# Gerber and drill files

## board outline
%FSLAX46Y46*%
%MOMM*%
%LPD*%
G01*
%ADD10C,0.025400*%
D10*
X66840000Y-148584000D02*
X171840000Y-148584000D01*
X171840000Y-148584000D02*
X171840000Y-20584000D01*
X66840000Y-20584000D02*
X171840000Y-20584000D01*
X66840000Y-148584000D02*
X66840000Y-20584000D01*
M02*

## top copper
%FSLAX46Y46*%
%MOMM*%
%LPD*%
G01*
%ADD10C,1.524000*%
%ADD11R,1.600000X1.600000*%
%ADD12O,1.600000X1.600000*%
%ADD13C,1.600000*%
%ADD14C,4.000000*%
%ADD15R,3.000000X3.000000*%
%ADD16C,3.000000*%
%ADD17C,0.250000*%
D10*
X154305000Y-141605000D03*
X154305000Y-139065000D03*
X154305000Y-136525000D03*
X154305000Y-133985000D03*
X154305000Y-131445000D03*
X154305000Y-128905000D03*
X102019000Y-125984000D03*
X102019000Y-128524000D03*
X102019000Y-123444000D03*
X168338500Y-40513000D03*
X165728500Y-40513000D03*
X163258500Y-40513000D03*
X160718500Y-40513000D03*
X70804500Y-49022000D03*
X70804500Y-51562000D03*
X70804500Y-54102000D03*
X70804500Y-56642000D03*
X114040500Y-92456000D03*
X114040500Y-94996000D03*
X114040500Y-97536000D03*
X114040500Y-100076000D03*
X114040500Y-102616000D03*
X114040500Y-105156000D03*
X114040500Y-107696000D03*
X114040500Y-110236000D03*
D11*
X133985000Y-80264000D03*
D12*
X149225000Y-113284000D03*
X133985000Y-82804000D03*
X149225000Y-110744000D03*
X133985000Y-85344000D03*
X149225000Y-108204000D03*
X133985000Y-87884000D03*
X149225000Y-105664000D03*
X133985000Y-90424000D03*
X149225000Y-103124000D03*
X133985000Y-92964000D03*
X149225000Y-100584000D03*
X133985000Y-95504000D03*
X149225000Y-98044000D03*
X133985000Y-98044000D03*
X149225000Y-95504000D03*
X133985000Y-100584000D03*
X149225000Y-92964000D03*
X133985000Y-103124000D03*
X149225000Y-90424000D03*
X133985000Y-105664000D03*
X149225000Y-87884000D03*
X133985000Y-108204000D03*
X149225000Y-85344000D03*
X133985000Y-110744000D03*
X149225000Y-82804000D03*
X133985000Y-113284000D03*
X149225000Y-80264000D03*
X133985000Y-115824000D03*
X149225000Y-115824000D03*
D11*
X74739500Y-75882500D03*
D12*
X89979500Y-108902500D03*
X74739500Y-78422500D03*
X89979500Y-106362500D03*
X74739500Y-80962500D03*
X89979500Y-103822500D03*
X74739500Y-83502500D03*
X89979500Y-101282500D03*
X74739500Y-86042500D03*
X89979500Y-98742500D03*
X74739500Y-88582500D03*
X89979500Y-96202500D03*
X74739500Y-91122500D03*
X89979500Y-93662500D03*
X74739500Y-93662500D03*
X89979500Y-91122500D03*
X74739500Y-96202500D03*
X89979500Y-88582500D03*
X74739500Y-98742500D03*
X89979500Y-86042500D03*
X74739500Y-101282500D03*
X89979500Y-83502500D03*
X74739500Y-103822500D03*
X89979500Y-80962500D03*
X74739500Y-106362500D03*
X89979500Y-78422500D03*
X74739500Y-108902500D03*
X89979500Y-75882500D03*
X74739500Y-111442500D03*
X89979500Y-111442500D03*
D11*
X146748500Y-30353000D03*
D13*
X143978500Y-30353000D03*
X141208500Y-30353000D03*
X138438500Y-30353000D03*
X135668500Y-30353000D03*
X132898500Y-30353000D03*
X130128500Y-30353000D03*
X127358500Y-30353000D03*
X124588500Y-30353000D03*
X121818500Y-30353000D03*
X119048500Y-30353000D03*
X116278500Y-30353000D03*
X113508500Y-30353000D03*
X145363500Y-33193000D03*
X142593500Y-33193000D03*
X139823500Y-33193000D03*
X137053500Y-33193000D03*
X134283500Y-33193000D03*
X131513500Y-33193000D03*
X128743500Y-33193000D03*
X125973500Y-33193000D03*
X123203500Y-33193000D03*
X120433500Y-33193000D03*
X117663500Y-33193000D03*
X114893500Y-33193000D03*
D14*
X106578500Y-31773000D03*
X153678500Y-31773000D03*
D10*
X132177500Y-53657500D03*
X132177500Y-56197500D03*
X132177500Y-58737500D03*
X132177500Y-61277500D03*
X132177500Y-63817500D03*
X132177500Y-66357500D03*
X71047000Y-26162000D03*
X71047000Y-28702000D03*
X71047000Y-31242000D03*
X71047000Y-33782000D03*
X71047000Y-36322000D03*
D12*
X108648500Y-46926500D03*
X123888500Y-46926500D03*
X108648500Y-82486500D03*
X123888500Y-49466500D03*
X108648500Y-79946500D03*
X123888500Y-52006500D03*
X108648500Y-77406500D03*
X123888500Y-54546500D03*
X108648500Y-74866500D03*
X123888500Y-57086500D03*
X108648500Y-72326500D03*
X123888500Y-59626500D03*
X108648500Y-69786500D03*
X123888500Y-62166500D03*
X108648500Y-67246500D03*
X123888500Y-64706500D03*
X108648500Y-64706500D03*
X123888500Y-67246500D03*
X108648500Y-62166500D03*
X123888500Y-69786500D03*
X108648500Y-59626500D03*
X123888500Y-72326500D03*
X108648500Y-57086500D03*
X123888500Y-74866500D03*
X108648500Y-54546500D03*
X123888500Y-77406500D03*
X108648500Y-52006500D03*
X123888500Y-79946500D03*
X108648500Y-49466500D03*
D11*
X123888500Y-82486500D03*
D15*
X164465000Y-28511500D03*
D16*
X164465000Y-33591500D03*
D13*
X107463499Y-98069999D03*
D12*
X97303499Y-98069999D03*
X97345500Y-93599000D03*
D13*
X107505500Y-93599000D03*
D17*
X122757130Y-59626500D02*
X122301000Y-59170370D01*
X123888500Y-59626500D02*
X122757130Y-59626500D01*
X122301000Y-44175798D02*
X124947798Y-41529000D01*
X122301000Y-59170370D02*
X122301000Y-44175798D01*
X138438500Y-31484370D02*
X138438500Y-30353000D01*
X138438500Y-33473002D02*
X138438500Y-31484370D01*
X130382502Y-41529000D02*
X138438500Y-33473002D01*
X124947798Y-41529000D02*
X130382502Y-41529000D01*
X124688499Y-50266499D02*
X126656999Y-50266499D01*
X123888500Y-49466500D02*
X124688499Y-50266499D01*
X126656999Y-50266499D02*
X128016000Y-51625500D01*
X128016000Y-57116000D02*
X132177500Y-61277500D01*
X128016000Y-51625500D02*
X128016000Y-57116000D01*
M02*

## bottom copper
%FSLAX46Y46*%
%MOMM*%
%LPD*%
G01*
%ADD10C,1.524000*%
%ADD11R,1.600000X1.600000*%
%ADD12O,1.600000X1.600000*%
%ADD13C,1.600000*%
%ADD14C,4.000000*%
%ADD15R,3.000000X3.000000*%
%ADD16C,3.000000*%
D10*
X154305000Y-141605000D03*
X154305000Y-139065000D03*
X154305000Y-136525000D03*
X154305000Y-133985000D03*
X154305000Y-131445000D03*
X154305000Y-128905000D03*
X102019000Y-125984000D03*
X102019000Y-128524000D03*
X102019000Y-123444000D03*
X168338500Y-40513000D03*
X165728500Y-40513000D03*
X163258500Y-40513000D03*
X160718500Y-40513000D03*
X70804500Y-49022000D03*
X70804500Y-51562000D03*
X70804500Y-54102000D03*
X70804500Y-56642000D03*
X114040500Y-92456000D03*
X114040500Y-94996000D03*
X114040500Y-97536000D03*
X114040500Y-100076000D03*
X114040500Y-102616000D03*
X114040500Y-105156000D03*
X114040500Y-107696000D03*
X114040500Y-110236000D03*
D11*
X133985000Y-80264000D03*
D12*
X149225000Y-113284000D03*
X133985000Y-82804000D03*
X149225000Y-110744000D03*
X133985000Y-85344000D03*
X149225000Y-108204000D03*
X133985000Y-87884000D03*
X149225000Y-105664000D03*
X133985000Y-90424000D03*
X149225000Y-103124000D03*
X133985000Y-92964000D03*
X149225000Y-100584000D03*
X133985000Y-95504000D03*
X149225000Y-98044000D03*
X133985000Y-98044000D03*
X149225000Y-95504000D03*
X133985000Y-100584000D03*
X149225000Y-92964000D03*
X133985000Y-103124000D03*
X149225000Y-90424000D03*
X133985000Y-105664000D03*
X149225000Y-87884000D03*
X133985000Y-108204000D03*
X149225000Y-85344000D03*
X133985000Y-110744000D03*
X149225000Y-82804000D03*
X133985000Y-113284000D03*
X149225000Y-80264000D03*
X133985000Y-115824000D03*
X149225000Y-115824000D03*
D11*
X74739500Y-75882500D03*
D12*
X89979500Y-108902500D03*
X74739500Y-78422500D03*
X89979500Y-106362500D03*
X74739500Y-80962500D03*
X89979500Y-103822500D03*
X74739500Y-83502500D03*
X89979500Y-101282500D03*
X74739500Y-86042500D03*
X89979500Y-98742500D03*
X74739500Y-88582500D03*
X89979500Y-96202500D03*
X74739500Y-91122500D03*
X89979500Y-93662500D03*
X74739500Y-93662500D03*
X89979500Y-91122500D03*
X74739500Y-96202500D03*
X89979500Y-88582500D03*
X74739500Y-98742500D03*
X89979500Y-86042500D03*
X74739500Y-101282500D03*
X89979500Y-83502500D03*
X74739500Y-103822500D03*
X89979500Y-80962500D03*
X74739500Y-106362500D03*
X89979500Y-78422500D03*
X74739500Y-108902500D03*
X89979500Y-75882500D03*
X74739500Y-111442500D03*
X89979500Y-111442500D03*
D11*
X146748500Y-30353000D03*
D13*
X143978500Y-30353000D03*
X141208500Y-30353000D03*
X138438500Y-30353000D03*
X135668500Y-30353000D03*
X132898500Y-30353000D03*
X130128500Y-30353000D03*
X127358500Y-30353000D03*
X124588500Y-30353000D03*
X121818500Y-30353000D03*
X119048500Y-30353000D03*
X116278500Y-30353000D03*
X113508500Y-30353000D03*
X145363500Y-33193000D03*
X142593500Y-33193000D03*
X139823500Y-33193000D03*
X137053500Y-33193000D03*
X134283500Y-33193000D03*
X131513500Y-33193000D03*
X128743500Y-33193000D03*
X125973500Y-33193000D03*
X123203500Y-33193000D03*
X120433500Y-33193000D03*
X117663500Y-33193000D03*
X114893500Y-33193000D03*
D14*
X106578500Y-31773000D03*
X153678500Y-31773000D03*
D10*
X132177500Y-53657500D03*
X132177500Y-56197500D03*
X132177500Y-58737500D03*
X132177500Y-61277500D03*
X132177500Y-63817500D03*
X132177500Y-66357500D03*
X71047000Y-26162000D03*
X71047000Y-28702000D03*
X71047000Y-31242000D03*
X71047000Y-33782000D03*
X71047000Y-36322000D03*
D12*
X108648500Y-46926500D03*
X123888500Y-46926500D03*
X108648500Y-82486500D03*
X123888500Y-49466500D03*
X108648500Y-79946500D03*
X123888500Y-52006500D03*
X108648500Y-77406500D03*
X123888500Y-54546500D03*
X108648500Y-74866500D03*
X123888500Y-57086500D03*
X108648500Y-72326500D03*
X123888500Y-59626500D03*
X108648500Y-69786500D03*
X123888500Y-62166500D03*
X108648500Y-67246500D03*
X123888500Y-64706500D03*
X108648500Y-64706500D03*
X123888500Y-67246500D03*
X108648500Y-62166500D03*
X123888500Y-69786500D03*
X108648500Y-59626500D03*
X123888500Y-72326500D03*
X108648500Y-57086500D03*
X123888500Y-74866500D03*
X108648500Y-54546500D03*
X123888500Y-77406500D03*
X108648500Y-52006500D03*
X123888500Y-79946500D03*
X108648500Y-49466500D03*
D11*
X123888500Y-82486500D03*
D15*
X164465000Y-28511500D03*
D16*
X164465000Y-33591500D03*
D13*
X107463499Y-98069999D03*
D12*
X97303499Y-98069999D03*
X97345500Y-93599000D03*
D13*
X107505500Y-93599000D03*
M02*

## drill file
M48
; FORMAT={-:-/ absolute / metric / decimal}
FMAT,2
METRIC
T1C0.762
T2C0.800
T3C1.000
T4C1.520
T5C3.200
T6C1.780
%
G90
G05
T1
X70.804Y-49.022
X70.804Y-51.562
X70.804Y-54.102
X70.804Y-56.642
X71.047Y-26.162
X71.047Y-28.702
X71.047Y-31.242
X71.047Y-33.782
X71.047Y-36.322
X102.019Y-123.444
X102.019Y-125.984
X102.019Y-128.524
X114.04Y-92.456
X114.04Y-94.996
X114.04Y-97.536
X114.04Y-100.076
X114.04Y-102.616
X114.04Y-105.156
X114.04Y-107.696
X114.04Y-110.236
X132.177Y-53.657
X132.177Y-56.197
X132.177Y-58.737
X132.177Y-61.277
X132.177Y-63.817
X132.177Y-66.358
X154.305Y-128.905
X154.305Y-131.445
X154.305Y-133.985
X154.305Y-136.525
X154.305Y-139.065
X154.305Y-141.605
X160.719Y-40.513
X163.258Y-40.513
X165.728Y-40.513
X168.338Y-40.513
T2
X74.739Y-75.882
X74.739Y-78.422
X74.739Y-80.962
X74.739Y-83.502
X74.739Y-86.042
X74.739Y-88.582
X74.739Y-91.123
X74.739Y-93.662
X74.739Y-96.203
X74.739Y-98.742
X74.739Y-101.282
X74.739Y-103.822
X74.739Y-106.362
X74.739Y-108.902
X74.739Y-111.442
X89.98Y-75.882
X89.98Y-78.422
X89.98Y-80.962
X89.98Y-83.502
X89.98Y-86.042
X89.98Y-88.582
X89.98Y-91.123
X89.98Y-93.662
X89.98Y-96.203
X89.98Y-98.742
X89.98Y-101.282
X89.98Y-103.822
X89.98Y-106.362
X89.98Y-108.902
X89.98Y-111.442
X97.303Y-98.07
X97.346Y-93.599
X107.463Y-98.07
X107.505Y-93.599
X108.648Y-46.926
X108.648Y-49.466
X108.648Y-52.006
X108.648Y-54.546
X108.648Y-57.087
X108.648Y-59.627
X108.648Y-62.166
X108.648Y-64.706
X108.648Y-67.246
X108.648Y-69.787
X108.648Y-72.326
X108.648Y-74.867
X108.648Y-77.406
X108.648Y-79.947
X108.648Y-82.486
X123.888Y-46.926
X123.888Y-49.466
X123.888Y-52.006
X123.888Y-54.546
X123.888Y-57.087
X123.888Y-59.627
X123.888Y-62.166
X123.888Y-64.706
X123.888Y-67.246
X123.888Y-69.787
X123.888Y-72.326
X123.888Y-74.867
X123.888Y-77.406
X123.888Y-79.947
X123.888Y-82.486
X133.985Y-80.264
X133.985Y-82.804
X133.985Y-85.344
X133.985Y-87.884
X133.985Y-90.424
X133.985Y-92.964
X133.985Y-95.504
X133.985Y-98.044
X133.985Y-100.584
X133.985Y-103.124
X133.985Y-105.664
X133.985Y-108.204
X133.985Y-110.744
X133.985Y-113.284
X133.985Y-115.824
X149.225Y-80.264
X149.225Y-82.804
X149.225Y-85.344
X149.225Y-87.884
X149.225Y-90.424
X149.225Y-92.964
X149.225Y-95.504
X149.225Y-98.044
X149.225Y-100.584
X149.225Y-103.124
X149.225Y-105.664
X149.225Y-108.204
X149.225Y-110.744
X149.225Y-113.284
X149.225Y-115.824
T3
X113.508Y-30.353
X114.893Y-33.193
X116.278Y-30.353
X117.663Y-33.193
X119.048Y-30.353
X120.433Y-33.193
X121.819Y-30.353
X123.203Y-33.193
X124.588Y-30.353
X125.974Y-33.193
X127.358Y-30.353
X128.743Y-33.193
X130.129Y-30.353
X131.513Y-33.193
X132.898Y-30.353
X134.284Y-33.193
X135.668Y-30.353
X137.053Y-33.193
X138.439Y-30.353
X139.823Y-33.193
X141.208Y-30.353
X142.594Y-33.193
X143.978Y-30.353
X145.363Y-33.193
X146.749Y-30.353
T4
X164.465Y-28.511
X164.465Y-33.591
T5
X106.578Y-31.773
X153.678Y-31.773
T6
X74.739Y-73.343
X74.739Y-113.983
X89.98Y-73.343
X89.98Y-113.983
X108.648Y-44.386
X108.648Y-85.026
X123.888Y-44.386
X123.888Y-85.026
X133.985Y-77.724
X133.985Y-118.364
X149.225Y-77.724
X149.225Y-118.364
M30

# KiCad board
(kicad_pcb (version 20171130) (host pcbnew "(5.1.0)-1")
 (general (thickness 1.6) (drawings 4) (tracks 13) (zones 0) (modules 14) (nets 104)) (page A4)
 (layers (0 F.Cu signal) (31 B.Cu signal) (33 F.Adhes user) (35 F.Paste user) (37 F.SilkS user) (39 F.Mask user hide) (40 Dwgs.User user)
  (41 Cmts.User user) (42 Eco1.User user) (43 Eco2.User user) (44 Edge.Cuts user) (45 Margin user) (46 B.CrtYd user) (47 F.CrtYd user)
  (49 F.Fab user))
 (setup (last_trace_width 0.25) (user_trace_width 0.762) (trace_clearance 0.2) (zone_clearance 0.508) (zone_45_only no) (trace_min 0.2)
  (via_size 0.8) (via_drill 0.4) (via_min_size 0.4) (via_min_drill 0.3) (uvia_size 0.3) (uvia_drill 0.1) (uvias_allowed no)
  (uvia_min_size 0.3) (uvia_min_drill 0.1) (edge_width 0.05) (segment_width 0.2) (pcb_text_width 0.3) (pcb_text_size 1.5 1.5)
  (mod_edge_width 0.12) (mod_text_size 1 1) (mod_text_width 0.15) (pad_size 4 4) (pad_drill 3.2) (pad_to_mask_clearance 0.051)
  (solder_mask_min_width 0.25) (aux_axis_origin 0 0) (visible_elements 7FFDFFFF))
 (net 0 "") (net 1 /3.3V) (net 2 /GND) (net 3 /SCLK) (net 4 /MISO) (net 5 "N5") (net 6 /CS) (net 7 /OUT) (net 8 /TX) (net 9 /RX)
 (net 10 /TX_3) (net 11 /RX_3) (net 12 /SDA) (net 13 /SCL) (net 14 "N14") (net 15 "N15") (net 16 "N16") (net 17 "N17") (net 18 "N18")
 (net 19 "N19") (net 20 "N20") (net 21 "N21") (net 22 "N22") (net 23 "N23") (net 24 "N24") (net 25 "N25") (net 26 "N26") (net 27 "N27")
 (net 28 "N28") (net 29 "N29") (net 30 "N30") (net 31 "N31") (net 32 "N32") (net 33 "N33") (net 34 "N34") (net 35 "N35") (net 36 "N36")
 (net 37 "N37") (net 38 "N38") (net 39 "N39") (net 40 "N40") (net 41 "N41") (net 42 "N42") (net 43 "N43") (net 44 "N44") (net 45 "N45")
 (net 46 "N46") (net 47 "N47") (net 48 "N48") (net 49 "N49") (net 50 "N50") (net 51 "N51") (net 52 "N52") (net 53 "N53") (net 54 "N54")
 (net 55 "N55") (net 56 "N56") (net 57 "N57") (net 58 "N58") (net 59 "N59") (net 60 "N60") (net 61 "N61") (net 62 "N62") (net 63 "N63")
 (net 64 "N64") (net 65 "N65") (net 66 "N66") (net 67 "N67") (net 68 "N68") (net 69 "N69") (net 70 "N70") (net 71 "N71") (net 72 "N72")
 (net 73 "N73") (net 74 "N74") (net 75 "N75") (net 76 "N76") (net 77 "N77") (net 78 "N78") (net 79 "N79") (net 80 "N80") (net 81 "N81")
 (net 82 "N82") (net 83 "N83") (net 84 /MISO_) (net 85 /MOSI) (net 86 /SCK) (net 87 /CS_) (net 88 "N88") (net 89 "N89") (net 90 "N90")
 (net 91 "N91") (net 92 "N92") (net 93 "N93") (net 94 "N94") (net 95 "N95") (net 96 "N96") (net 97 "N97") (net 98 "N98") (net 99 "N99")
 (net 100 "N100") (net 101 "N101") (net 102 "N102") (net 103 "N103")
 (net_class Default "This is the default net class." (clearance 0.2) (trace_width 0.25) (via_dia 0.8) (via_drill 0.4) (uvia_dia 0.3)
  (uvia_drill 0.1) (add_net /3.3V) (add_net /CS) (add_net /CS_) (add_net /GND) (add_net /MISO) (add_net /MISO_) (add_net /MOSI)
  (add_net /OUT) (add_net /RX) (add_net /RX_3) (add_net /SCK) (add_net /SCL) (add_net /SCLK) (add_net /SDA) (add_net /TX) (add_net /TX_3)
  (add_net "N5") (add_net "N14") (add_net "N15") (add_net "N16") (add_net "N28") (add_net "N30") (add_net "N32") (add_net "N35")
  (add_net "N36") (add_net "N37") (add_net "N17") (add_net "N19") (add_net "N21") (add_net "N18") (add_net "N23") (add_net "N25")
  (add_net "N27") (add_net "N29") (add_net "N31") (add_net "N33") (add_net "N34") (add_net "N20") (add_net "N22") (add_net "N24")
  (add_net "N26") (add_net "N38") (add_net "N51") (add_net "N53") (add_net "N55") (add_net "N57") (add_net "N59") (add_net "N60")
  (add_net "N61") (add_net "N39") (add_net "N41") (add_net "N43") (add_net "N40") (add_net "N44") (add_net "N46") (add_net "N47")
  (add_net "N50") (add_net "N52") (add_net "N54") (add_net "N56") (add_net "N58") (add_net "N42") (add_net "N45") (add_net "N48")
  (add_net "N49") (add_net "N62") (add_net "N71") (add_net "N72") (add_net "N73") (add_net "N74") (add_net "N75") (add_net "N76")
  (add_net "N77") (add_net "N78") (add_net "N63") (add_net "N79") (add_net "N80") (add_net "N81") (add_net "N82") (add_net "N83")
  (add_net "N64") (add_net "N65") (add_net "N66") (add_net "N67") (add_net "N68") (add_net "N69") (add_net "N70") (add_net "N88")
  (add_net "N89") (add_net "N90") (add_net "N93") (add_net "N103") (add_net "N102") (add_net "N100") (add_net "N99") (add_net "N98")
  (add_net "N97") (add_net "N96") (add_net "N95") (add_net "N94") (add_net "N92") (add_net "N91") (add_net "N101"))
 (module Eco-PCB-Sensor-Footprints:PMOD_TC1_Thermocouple (layer F.Cu) (at 150.495 137.795 90)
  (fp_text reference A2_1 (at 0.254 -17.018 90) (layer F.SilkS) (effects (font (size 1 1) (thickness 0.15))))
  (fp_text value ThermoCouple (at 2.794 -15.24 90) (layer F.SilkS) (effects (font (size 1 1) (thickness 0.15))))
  (pad 1 thru_hole circle (at -3.81 3.81 90) (size 1.524 1.524) (drill 0.762) (layers *.Cu *.Mask) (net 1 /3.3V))
  (pad 2 thru_hole circle (at -1.27 3.81 90) (size 1.524 1.524) (drill 0.762) (layers *.Cu *.Mask) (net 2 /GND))
  (pad 3 thru_hole circle (at 1.27 3.81 90) (size 1.524 1.524) (drill 0.762) (layers *.Cu *.Mask) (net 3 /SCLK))
  (pad 4 thru_hole circle (at 3.81 3.81 90) (size 1.524 1.524) (drill 0.762) (layers *.Cu *.Mask) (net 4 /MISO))
  (pad 5 thru_hole circle (at 6.35 3.81 90) (size 1.524 1.524) (drill 0.762) (layers *.Cu *.Mask) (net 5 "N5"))
  (pad 6 thru_hole circle (at 8.89 3.81 90) (size 1.524 1.524) (drill 0.762) (layers *.Cu *.Mask) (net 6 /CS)))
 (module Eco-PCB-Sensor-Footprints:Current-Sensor (layer F.Cu) (at 88.519 125.984 90)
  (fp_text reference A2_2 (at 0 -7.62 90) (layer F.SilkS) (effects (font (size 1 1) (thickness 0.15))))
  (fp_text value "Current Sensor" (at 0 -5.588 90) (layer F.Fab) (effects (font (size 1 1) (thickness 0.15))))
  (pad 2 thru_hole circle (at 0 13.5 90) (size 1.524 1.524) (drill 0.762) (layers *.Cu *.Mask) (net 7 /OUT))
  (pad 1 thru_hole circle (at -2.54 13.5 90) (size 1.524 1.524) (drill 0.762) (layers *.Cu *.Mask) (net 1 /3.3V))
  (pad 3 thru_hole circle (at 2.54 13.5 90) (size 1.524 1.524) (drill 0.762) (layers *.Cu *.Mask) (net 2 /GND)))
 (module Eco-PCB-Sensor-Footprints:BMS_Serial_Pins (layer F.Cu) (at 164.5285 40.513 180)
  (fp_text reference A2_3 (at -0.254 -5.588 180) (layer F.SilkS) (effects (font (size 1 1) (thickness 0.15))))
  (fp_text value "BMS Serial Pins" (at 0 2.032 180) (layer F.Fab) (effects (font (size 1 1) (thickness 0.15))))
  (pad 1 thru_hole circle (at -3.81 0 180) (size 1.524 1.524) (drill 0.762) (layers *.Cu *.Mask) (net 1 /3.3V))
  (pad 2 thru_hole circle (at -1.2 0 180) (size 1.524 1.524) (drill 0.762) (layers *.Cu *.Mask) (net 2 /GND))
  (pad 3 thru_hole circle (at 1.27 0 180) (size 1.524 1.524) (drill 0.762) (layers *.Cu *.Mask) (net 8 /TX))
  (pad 4 thru_hole circle (at 3.81 0 180) (size 1.524 1.524) (drill 0.762) (layers *.Cu *.Mask) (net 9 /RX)))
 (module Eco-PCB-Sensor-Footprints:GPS (layer F.Cu) (at 86.8045 52.832 270)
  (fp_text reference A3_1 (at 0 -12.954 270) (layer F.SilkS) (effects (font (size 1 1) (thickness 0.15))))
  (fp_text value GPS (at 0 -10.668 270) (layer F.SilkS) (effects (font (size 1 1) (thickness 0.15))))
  (pad 1 thru_hole circle (at -3.81 16 270) (size 1.524 1.524) (drill 0.762) (layers *.Cu *.Mask) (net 2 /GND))
  (pad 2 thru_hole circle (at -1.27 16 270) (size 1.524 1.524) (drill 0.762) (layers *.Cu *.Mask) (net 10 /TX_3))
  (pad 3 thru_hole circle (at 1.27 16 270) (size 1.524 1.524) (drill 0.762) (layers *.Cu *.Mask) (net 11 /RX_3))
  (pad 4 thru_hole circle (at 3.81 16 270) (size 1.524 1.524) (drill 0.762) (layers *.Cu *.Mask) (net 1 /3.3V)))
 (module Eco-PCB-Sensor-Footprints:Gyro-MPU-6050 (layer F.Cu) (at 120.8405 101.346 270)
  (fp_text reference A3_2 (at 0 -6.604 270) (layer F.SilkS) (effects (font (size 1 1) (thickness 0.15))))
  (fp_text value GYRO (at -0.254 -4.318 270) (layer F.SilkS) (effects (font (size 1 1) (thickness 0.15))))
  (pad 1 thru_hole circle (at -8.89 6.8 270) (size 1.524 1.524) (drill 0.762) (layers *.Cu *.Mask) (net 1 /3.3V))
  (pad 2 thru_hole circle (at -6.35 6.8 270) (size 1.524 1.524) (drill 0.762) (layers *.Cu *.Mask) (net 2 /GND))
  (pad 3 thru_hole circle (at -3.81 6.8 270) (size 1.524 1.524) (drill 0.762) (layers *.Cu *.Mask) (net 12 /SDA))
  (pad 4 thru_hole circle (at -1.27 6.8 270) (size 1.524 1.524) (drill 0.762) (layers *.Cu *.Mask) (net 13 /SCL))
  (pad 5 thru_hole circle (at 1.27 6.8 270) (size 1.524 1.524) (drill 0.762) (layers *.Cu *.Mask) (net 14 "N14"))
  (pad 6 thru_hole circle (at 3.81 6.8 270) (size 1.524 1.524) (drill 0.762) (layers *.Cu *.Mask) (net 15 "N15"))
  (pad 7 thru_hole circle (at 6.35 6.8 270) (size 1.524 1.524) (drill 0.762) (layers *.Cu *.Mask))
  (pad 8 thru_hole circle (at 8.89 6.8 270) (size 1.524 1.524) (drill 0.762) (layers *.Cu *.Mask)))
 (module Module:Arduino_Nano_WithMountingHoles (layer F.Cu) (at 133.985 80.264)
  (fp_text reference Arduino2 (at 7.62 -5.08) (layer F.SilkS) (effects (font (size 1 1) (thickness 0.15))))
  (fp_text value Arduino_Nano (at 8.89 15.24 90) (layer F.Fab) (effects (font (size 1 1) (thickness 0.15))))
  (pad 1 thru_hole rect (at 0 0) (size 1.6 1.6) (drill 0.8) (layers *.Cu *.Mask) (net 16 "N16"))
  (pad 17 thru_hole oval (at 15.24 33.02) (size 1.6 1.6) (drill 0.8) (layers *.Cu *.Mask) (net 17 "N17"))
  (pad 2 thru_hole oval (at 0 2.54) (size 1.6 1.6) (drill 0.8) (layers *.Cu *.Mask) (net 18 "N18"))
  (pad 18 thru_hole oval (at 15.24 30.48) (size 1.6 1.6) (drill 0.8) (layers *.Cu *.Mask) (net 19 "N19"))
  (pad 3 thru_hole oval (at 0 5.08) (size 1.6 1.6) (drill 0.8) (layers *.Cu *.Mask) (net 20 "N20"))
  (pad 19 thru_hole oval (at 15.24 27.94) (size 1.6 1.6) (drill 0.8) (layers *.Cu *.Mask) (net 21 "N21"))
  (pad 4 thru_hole oval (at 0 7.62) (size 1.6 1.6) (drill 0.8) (layers *.Cu *.Mask) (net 2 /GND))
  (pad 20 thru_hole oval (at 15.24 25.4) (size 1.6 1.6) (drill 0.8) (layers *.Cu *.Mask) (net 7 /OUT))
  (pad 5 thru_hole oval (at 0 10.16) (size 1.6 1.6) (drill 0.8) (layers *.Cu *.Mask) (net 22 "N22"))
  (pad 21 thru_hole oval (at 15.24 22.86) (size 1.6 1.6) (drill 0.8) (layers *.Cu *.Mask) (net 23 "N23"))
  (pad 6 thru_hole oval (at 0 12.7) (size 1.6 1.6) (drill 0.8) (layers *.Cu *.Mask) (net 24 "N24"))
  (pad 22 thru_hole oval (at 15.24 20.32) (size 1.6 1.6) (drill 0.8) (layers *.Cu *.Mask) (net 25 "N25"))
  (pad 7 thru_hole oval (at 0 15.24) (size 1.6 1.6) (drill 0.8) (layers *.Cu *.Mask) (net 8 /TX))
  (pad 23 thru_hole oval (at 15.24 17.78) (size 1.6 1.6) (drill 0.8) (layers *.Cu *.Mask) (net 6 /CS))
  (pad 8 thru_hole oval (at 0 17.78) (size 1.6 1.6) (drill 0.8) (layers *.Cu *.Mask) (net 9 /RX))
  (pad 24 thru_hole oval (at 15.24 15.24) (size 1.6 1.6) (drill 0.8) (layers *.Cu *.Mask) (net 4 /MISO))
  (pad 9 thru_hole oval (at 0 20.32) (size 1.6 1.6) (drill 0.8) (layers *.Cu *.Mask) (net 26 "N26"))
  (pad 25 thru_hole oval (at 15.24 12.7) (size 1.6 1.6) (drill 0.8) (layers *.Cu *.Mask) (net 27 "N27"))
  (pad 10 thru_hole oval (at 0 22.86) (size 1.6 1.6) (drill 0.8) (layers *.Cu *.Mask) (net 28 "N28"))
  (pad 26 thru_hole oval (at 15.24 10.16) (size 1.6 1.6) (drill 0.8) (layers *.Cu *.Mask) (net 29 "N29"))
  (pad 11 thru_hole oval (at 0 25.4) (size 1.6 1.6) (drill 0.8) (layers *.Cu *.Mask) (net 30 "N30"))
  (pad 27 thru_hole oval (at 15.24 7.62) (size 1.6 1.6) (drill 0.8) (layers *.Cu *.Mask) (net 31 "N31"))
  (pad 12 thru_hole oval (at 0 27.94) (size 1.6 1.6) (drill 0.8) (layers *.Cu *.Mask) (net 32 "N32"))
  (pad 28 thru_hole oval (at 15.24 5.08) (size 1.6 1.6) (drill 0.8) (layers *.Cu *.Mask) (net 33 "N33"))
  (pad 13 thru_hole oval (at 0 30.48) (size 1.6 1.6) (drill 0.8) (layers *.Cu *.Mask) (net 3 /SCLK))
  (pad 29 thru_hole oval (at 15.24 2.54) (size 1.6 1.6) (drill 0.8) (layers *.Cu *.Mask) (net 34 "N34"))
  (pad 14 thru_hole oval (at 0 33.02) (size 1.6 1.6) (drill 0.8) (layers *.Cu *.Mask) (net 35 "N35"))
  (pad 30 thru_hole oval (at 15.24 0) (size 1.6 1.6) (drill 0.8) (layers *.Cu *.Mask) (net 1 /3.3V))
  (pad 15 thru_hole oval (at 0 35.56) (size 1.6 1.6) (drill 0.8) (layers *.Cu *.Mask) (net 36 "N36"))
  (pad 16 thru_hole oval (at 15.24 35.56) (size 1.6 1.6) (drill 0.8) (layers *.Cu *.Mask) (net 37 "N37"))
  (pad "" np_thru_hole circle (at 0 -2.54) (size 1.78 1.78) (drill 1.78) (layers *.Cu *.Mask))
  (pad "" np_thru_hole circle (at 15.24 -2.54) (size 1.78 1.78) (drill 1.78) (layers *.Cu *.Mask))
  (pad "" np_thru_hole circle (at 15.24 38.1) (size 1.78 1.78) (drill 1.78) (layers *.Cu *.Mask))
  (pad "" np_thru_hole circle (at 0 38.1) (size 1.78 1.78) (drill 1.78) (layers *.Cu *.Mask)))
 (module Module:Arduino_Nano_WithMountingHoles (layer F.Cu) (at 74.7395 75.8825)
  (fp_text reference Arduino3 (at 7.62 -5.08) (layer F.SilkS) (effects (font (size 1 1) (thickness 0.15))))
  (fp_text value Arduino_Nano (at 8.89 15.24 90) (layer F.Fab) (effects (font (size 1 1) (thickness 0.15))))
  (pad 1 thru_hole rect (at 0 0) (size 1.6 1.6) (drill 0.8) (layers *.Cu *.Mask) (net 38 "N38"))
  (pad 17 thru_hole oval (at 15.24 33.02) (size 1.6 1.6) (drill 0.8) (layers *.Cu *.Mask) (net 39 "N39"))
  (pad 2 thru_hole oval (at 0 2.54) (size 1.6 1.6) (drill 0.8) (layers *.Cu *.Mask) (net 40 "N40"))
  (pad 18 thru_hole oval (at 15.24 30.48) (size 1.6 1.6) (drill 0.8) (layers *.Cu *.Mask) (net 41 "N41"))
  (pad 3 thru_hole oval (at 0 5.08) (size 1.6 1.6) (drill 0.8) (layers *.Cu *.Mask) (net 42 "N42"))
  (pad 19 thru_hole oval (at 15.24 27.94) (size 1.6 1.6) (drill 0.8) (layers *.Cu *.Mask) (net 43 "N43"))
  (pad 4 thru_hole oval (at 0 7.62) (size 1.6 1.6) (drill 0.8) (layers *.Cu *.Mask) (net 2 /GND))
  (pad 20 thru_hole oval (at 15.24 25.4) (size 1.6 1.6) (drill 0.8) (layers *.Cu *.Mask) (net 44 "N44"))
  (pad 5 thru_hole oval (at 0 10.16) (size 1.6 1.6) (drill 0.8) (layers *.Cu *.Mask) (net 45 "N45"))
  (pad 21 thru_hole oval (at 15.24 22.86) (size 1.6 1.6) (drill 0.8) (layers *.Cu *.Mask) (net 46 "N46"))
  (pad 6 thru_hole oval (at 0 12.7) (size 1.6 1.6) (drill 0.8) (layers *.Cu *.Mask) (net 11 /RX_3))
  (pad 22 thru_hole oval (at 15.24 20.32) (size 1.6 1.6) (drill 0.8) (layers *.Cu *.Mask) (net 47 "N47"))
  (pad 7 thru_hole oval (at 0 15.24) (size 1.6 1.6) (drill 0.8) (layers *.Cu *.Mask) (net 10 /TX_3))
  (pad 23 thru_hole oval (at 15.24 17.78) (size 1.6 1.6) (drill 0.8) (layers *.Cu *.Mask) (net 13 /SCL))
  (pad 8 thru_hole oval (at 0 17.78) (size 1.6 1.6) (drill 0.8) (layers *.Cu *.Mask) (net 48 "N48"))
  (pad 24 thru_hole oval (at 15.24 15.24) (size 1.6 1.6) (drill 0.8) (layers *.Cu *.Mask) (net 12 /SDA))
  (pad 9 thru_hole oval (at 0 20.32) (size 1.6 1.6) (drill 0.8) (layers *.Cu *.Mask) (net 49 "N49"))
  (pad 25 thru_hole oval (at 15.24 12.7) (size 1.6 1.6) (drill 0.8) (layers *.Cu *.Mask) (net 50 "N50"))
  (pad 10 thru_hole oval (at 0 22.86) (size 1.6 1.6) (drill 0.8) (layers *.Cu *.Mask) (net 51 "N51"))
  (pad 26 thru_hole oval (at 15.24 10.16) (size 1.6 1.6) (drill 0.8) (layers *.Cu *.Mask) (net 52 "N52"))
  (pad 11 thru_hole oval (at 0 25.4) (size 1.6 1.6) (drill 0.8) (layers *.Cu *.Mask) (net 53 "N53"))
  (pad 27 thru_hole oval (at 15.24 7.62) (size 1.6 1.6) (drill 0.8) (layers *.Cu *.Mask) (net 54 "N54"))
  (pad 12 thru_hole oval (at 0 27.94) (size 1.6 1.6) (drill 0.8) (layers *.Cu *.Mask) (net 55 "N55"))
  (pad 28 thru_hole oval (at 15.24 5.08) (size 1.6 1.6) (drill 0.8) (layers *.Cu *.Mask) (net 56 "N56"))
  (pad 13 thru_hole oval (at 0 30.48) (size 1.6 1.6) (drill 0.8) (layers *.Cu *.Mask) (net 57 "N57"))
  (pad 29 thru_hole oval (at 15.24 2.54) (size 1.6 1.6) (drill 0.8) (layers *.Cu *.Mask) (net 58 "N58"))
  (pad 14 thru_hole oval (at 0 33.02) (size 1.6 1.6) (drill 0.8) (layers *.Cu *.Mask) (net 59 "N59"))
  (pad 30 thru_hole oval (at 15.24 0) (size 1.6 1.6) (drill 0.8) (layers *.Cu *.Mask) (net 1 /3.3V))
  (pad 15 thru_hole oval (at 0 35.56) (size 1.6 1.6) (drill 0.8) (layers *.Cu *.Mask) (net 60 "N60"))
  (pad 16 thru_hole oval (at 15.24 35.56) (size 1.6 1.6) (drill 0.8) (layers *.Cu *.Mask) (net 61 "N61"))
  (pad "" np_thru_hole circle (at 0 -2.54) (size 1.78 1.78) (drill 1.78) (layers *.Cu *.Mask))
  (pad "" np_thru_hole circle (at 15.24 -2.54) (size 1.78 1.78) (drill 1.78) (layers *.Cu *.Mask))
  (pad "" np_thru_hole circle (at 15.24 38.1) (size 1.78 1.78) (drill 1.78) (layers *.Cu *.Mask))
  (pad "" np_thru_hole circle (at 0 38.1) (size 1.78 1.78) (drill 1.78) (layers *.Cu *.Mask)))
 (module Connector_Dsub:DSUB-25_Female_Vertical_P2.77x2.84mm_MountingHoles (layer F.Cu) (at 146.7485 30.353)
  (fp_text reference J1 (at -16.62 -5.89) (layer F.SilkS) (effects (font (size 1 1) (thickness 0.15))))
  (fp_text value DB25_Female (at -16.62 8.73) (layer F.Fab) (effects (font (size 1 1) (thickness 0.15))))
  (pad 1 thru_hole rect (at 0 0) (size 1.6 1.6) (drill 1) (layers *.Cu *.Mask) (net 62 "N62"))
  (pad 2 thru_hole circle (at -2.77 0) (size 1.6 1.6) (drill 1) (layers *.Cu *.Mask) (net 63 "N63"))
  (pad 3 thru_hole circle (at -5.54 0) (size 1.6 1.6) (drill 1) (layers *.Cu *.Mask) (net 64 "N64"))
  (pad 4 thru_hole circle (at -8.31 0) (size 1.6 1.6) (drill 1) (layers *.Cu *.Mask) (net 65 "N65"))
  (pad 5 thru_hole circle (at -11.08 0) (size 1.6 1.6) (drill 1) (layers *.Cu *.Mask) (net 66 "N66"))
  (pad 6 thru_hole circle (at -13.85 0) (size 1.6 1.6) (drill 1) (layers *.Cu *.Mask) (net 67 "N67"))
  (pad 7 thru_hole circle (at -16.62 0) (size 1.6 1.6) (drill 1) (layers *.Cu *.Mask) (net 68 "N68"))
  (pad 8 thru_hole circle (at -19.39 0) (size 1.6 1.6) (drill 1) (layers *.Cu *.Mask) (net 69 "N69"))
  (pad 9 thru_hole circle (at -22.16 0) (size 1.6 1.6) (drill 1) (layers *.Cu *.Mask) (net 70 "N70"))
  (pad 10 thru_hole circle (at -24.93 0) (size 1.6 1.6) (drill 1) (layers *.Cu *.Mask) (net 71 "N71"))
  (pad 11 thru_hole circle (at -27.7 0) (size 1.6 1.6) (drill 1) (layers *.Cu *.Mask) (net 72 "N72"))
  (pad 12 thru_hole circle (at -30.47 0) (size 1.6 1.6) (drill 1) (layers *.Cu *.Mask) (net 2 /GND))
  (pad 13 thru_hole circle (at -33.24 0) (size 1.6 1.6) (drill 1) (layers *.Cu *.Mask) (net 1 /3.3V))
  (pad 14 thru_hole circle (at -1.385 2.84) (size 1.6 1.6) (drill 1) (layers *.Cu *.Mask) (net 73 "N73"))
  (pad 15 thru_hole circle (at -4.155 2.84) (size 1.6 1.6) (drill 1) (layers *.Cu *.Mask) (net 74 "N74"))
  (pad 16 thru_hole circle (at -6.925 2.84) (size 1.6 1.6) (drill 1) (layers *.Cu *.Mask) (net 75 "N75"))
  (pad 17 thru_hole circle (at -9.695 2.84) (size 1.6 1.6) (drill 1) (layers *.Cu *.Mask) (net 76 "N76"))
  (pad 18 thru_hole circle (at -12.465 2.84) (size 1.6 1.6) (drill 1) (layers *.Cu *.Mask) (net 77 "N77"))
  (pad 19 thru_hole circle (at -15.235 2.84) (size 1.6 1.6) (drill 1) (layers *.Cu *.Mask) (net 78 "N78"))
  (pad 20 thru_hole circle (at -18.005 2.84) (size 1.6 1.6) (drill 1) (layers *.Cu *.Mask) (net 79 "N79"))
  (pad 21 thru_hole circle (at -20.775 2.84) (size 1.6 1.6) (drill 1) (layers *.Cu *.Mask) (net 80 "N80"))
  (pad 22 thru_hole circle (at -23.545 2.84) (size 1.6 1.6) (drill 1) (layers *.Cu *.Mask) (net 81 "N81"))
  (pad 23 thru_hole circle (at -26.315 2.84) (size 1.6 1.6) (drill 1) (layers *.Cu *.Mask) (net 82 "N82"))
  (pad 24 thru_hole circle (at -29.085 2.84) (size 1.6 1.6) (drill 1) (layers *.Cu *.Mask) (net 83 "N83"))
  (pad 25 thru_hole circle (at -31.855 2.84) (size 1.6 1.6) (drill 1) (layers *.Cu *.Mask) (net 1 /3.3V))
  (pad 0 thru_hole circle (at -40.17 1.42) (size 4 4) (drill 3.2) (layers *.Cu *.Mask) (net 2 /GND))
  (pad 0 thru_hole circle (at 6.93 1.42) (size 4 4) (drill 3.2) (layers *.Cu *.Mask) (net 2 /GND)))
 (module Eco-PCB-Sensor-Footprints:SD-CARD (layer F.Cu) (at 150.1775 60.0075 270)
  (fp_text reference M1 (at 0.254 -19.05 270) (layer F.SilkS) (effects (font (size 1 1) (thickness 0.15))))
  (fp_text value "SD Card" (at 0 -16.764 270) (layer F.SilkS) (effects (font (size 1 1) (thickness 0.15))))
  (pad 1 thru_hole circle (at -6.35 18 270) (size 1.524 1.524) (drill 0.762) (layers *.Cu *.Mask) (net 2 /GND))
  (pad 2 thru_hole circle (at -3.81 18 270) (size 1.524 1.524) (drill 0.762) (layers *.Cu *.Mask) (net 1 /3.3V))
  (pad 3 thru_hole circle (at -1.27 18 270) (size 1.524 1.524) (drill 0.762) (layers *.Cu *.Mask) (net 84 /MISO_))
  (pad 4 thru_hole circle (at 1.27 18) (size 1.524 1.524) (drill 0.762) (layers *.Cu *.Mask) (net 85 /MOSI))
  (pad 5 thru_hole circle (at 3.81 18 270) (size 1.524 1.524) (drill 0.762) (layers *.Cu *.Mask) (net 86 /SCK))
  (pad 6 thru_hole circle (at 6.35 18 270) (size 1.524 1.524) (drill 0.762) (layers *.Cu *.Mask) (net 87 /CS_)))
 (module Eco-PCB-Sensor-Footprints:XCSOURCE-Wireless (layer F.Cu) (at 83.947 31.242 270)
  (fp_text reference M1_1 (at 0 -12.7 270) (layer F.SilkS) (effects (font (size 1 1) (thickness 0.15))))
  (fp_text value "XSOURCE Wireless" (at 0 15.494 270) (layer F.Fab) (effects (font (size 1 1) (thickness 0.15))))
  (pad 1 thru_hole circle (at -5.08 12.9 270) (size 1.524 1.524) (drill 0.762) (layers *.Cu *.Mask) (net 1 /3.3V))
  (pad 2 thru_hole circle (at -2.54 12.9 270) (size 1.524 1.524) (drill 0.762) (layers *.Cu *.Mask) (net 2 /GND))
  (pad 3 thru_hole circle (at 0 12.9 270) (size 1.524 1.524) (drill 0.762) (layers *.Cu *.Mask) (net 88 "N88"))
  (pad 4 thru_hole circle (at 2.54 12.9 270) (size 1.524 1.524) (drill 0.762) (layers *.Cu *.Mask) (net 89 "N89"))
  (pad 5 thru_hole circle (at 5.08 12.9 270) (size 1.524 1.524) (drill 0.762) (layers *.Cu *.Mask) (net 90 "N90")))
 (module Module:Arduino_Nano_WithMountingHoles (layer F.Cu) (at 123.8885 82.4865 180)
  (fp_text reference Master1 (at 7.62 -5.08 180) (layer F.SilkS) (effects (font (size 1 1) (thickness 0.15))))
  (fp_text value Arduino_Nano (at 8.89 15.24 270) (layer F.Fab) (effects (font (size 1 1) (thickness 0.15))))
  (pad "" np_thru_hole circle (at 0 38.1 180) (size 1.78 1.78) (drill 1.78) (layers *.Cu *.Mask))
  (pad "" np_thru_hole circle (at 15.24 38.1 180) (size 1.78 1.78) (drill 1.78) (layers *.Cu *.Mask))
  (pad "" np_thru_hole circle (at 15.24 -2.54 180) (size 1.78 1.78) (drill 1.78) (layers *.Cu *.Mask))
  (pad "" np_thru_hole circle (at 0 -2.54 180) (size 1.78 1.78) (drill 1.78) (layers *.Cu *.Mask))
  (pad 16 thru_hole oval (at 15.24 35.56 180) (size 1.6 1.6) (drill 0.8) (layers *.Cu *.Mask) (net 86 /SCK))
  (pad 15 thru_hole oval (at 0 35.56 180) (size 1.6 1.6) (drill 0.8) (layers *.Cu *.Mask) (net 84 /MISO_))
  (pad 30 thru_hole oval (at 15.24 0 180) (size 1.6 1.6) (drill 0.8) (layers *.Cu *.Mask) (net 1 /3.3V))
  (pad 14 thru_hole oval (at 0 33.02 180) (size 1.6 1.6) (drill 0.8) (layers *.Cu *.Mask) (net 85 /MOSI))
  (pad 29 thru_hole oval (at 15.24 2.54 180) (size 1.6 1.6) (drill 0.8) (layers *.Cu *.Mask) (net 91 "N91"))
  (pad 13 thru_hole oval (at 0 30.48 180) (size 1.6 1.6) (drill 0.8) (layers *.Cu *.Mask) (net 87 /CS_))
  (pad 28 thru_hole oval (at 15.24 5.08 180) (size 1.6 1.6) (drill 0.8) (layers *.Cu *.Mask) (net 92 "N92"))
  (pad 12 thru_hole oval (at 0 27.94 180) (size 1.6 1.6) (drill 0.8) (layers *.Cu *.Mask) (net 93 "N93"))
  (pad 27 thru_hole oval (at 15.24 7.62 180) (size 1.6 1.6) (drill 0.8) (layers *.Cu *.Mask) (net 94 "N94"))
  (pad 11 thru_hole oval (at 0 25.4 180) (size 1.6 1.6) (drill 0.8) (layers *.Cu *.Mask) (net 73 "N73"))
  (pad 26 thru_hole oval (at 15.24 10.16 180) (size 1.6 1.6) (drill 0.8) (layers *.Cu *.Mask) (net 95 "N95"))
  (pad 10 thru_hole oval (at 0 22.86 180) (size 1.6 1.6) (drill 0.8) (layers *.Cu *.Mask) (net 65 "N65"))
  (pad 25 thru_hole oval (at 15.24 12.7 180) (size 1.6 1.6) (drill 0.8) (layers *.Cu *.Mask) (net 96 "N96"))
  (pad 9 thru_hole oval (at 0 20.32 180) (size 1.6 1.6) (drill 0.8) (layers *.Cu *.Mask) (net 64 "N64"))
  (pad 24 thru_hole oval (at 15.24 15.24 180) (size 1.6 1.6) (drill 0.8) (layers *.Cu *.Mask) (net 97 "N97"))
  (pad 8 thru_hole oval (at 0 17.78 180) (size 1.6 1.6) (drill 0.8) (layers *.Cu *.Mask) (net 63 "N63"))
  (pad 23 thru_hole oval (at 15.24 17.78 180) (size 1.6 1.6) (drill 0.8) (layers *.Cu *.Mask) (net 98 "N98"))
  (pad 7 thru_hole oval (at 0 15.24 180) (size 1.6 1.6) (drill 0.8) (layers *.Cu *.Mask) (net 62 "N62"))
  (pad 22 thru_hole oval (at 15.24 20.32 180) (size 1.6 1.6) (drill 0.8) (layers *.Cu *.Mask) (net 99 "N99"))
  (pad 6 thru_hole oval (at 0 12.7 180) (size 1.6 1.6) (drill 0.8) (layers *.Cu *.Mask) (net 67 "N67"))
  (pad 21 thru_hole oval (at 15.24 22.86 180) (size 1.6 1.6) (drill 0.8) (layers *.Cu *.Mask) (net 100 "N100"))
  (pad 5 thru_hole oval (at 0 10.16 180) (size 1.6 1.6) (drill 0.8) (layers *.Cu *.Mask) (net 66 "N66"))
  (pad 20 thru_hole oval (at 15.24 25.4 180) (size 1.6 1.6) (drill 0.8) (layers *.Cu *.Mask) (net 40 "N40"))
  (pad 4 thru_hole oval (at 0 7.62 180) (size 1.6 1.6) (drill 0.8) (layers *.Cu *.Mask) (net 2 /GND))
  (pad 19 thru_hole oval (at 15.24 27.94 180) (size 1.6 1.6) (drill 0.8) (layers *.Cu *.Mask) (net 38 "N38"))
  (pad 3 thru_hole oval (at 0 5.08 180) (size 1.6 1.6) (drill 0.8) (layers *.Cu *.Mask) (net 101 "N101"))
  (pad 18 thru_hole oval (at 15.24 30.48 180) (size 1.6 1.6) (drill 0.8) (layers *.Cu *.Mask) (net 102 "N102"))
  (pad 2 thru_hole oval (at 0 2.54 180) (size 1.6 1.6) (drill 0.8) (layers *.Cu *.Mask) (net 18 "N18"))
  (pad 17 thru_hole oval (at 15.24 33.02 180) (size 1.6 1.6) (drill 0.8) (layers *.Cu *.Mask) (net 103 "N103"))
  (pad 1 thru_hole rect (at 0 0 180) (size 1.6 1.6) (drill 0.8) (layers *.Cu *.Mask) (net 16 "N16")))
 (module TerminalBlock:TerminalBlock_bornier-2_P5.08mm (layer F.Cu) (at 164.465 28.5115 270)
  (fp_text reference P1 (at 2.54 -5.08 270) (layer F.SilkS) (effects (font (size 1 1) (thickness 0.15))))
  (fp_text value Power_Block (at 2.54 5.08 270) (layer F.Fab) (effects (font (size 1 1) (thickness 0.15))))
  (pad 1 thru_hole rect (at 0 0 270) (size 3 3) (drill 1.52) (layers *.Cu *.Mask) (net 1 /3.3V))
  (pad 2 thru_hole circle (at 5.08 0 270) (size 3 3) (drill 1.52) (layers *.Cu *.Mask) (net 2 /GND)))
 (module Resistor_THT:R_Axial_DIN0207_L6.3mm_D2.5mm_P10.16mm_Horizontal (layer F.Cu) (at 107.463499 98.069999 180)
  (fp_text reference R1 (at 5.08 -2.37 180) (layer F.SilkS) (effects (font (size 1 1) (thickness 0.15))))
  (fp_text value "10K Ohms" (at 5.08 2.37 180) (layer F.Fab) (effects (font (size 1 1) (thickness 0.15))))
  (pad 1 thru_hole circle (at 0 0 180) (size 1.6 1.6) (drill 0.8) (layers *.Cu *.Mask) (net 1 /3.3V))
  (pad 2 thru_hole oval (at 10.16 0 180) (size 1.6 1.6) (drill 0.8) (layers *.Cu *.Mask) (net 12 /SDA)))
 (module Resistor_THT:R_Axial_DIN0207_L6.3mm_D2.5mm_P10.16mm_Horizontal (layer F.Cu) (at 107.5055 93.599 180)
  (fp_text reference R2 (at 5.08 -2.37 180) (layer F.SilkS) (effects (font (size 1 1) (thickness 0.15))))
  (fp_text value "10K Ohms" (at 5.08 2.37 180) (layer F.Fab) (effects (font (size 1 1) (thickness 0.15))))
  (pad 2 thru_hole oval (at 10.16 0 180) (size 1.6 1.6) (drill 0.8) (layers *.Cu *.Mask) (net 13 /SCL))
  (pad 1 thru_hole circle (at 0 0 180) (size 1.6 1.6) (drill 0.8) (layers *.Cu *.Mask) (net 1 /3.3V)))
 (gr_line (start 66.84 148.584) (end 171.84 148.584) (layer Edge.Cuts) (width 0.0254))
 (gr_line (start 171.84 148.584) (end 171.84 20.584) (layer Edge.Cuts) (width 0.0254))
 (gr_line (start 66.84 20.584) (end 171.84 20.584) (layer Edge.Cuts) (width 0.0254))
 (gr_line (start 66.84 148.584) (end 66.84 20.584) (layer Edge.Cuts) (width 0.0254))
 (segment (start 122.75713 59.6265) (end 122.301 59.17037) (width 0.25) (layer F.Cu) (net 65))
 (segment (start 123.8885 59.6265) (end 122.75713 59.6265) (width 0.25) (layer F.Cu) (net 65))
 (segment (start 122.301 44.175798) (end 124.947798 41.529) (width 0.25) (layer F.Cu) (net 65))
 (segment (start 122.301 59.17037) (end 122.301 44.175798) (width 0.25) (layer F.Cu) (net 65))
 (segment (start 138.4385 31.48437) (end 138.4385 30.353) (width 0.25) (layer F.Cu) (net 65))
 (segment (start 138.4385 33.473002) (end 138.4385 31.48437) (width 0.25) (layer F.Cu) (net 65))
 (segment (start 130.382502 41.529) (end 138.4385 33.473002) (width 0.25) (layer F.Cu) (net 65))
 (segment (start 124.947798 41.529) (end 130.382502 41.529) (width 0.25) (layer F.Cu) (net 65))
 (segment (start 124.688499 50.266499) (end 126.656999 50.266499) (width 0.25) (layer F.Cu) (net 85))
 (segment (start 123.8885 49.4665) (end 124.688499 50.266499) (width 0.25) (layer F.Cu) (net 85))
 (segment (start 126.656999 50.266499) (end 128.016 51.6255) (width 0.25) (layer F.Cu) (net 85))
 (segment (start 128.016 57.116) (end 132.1775 61.2775) (width 0.25) (layer F.Cu) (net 85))
 (segment (start 128.016 51.6255) (end 128.016 57.116) (width 0.25) (layer F.Cu) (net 85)))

